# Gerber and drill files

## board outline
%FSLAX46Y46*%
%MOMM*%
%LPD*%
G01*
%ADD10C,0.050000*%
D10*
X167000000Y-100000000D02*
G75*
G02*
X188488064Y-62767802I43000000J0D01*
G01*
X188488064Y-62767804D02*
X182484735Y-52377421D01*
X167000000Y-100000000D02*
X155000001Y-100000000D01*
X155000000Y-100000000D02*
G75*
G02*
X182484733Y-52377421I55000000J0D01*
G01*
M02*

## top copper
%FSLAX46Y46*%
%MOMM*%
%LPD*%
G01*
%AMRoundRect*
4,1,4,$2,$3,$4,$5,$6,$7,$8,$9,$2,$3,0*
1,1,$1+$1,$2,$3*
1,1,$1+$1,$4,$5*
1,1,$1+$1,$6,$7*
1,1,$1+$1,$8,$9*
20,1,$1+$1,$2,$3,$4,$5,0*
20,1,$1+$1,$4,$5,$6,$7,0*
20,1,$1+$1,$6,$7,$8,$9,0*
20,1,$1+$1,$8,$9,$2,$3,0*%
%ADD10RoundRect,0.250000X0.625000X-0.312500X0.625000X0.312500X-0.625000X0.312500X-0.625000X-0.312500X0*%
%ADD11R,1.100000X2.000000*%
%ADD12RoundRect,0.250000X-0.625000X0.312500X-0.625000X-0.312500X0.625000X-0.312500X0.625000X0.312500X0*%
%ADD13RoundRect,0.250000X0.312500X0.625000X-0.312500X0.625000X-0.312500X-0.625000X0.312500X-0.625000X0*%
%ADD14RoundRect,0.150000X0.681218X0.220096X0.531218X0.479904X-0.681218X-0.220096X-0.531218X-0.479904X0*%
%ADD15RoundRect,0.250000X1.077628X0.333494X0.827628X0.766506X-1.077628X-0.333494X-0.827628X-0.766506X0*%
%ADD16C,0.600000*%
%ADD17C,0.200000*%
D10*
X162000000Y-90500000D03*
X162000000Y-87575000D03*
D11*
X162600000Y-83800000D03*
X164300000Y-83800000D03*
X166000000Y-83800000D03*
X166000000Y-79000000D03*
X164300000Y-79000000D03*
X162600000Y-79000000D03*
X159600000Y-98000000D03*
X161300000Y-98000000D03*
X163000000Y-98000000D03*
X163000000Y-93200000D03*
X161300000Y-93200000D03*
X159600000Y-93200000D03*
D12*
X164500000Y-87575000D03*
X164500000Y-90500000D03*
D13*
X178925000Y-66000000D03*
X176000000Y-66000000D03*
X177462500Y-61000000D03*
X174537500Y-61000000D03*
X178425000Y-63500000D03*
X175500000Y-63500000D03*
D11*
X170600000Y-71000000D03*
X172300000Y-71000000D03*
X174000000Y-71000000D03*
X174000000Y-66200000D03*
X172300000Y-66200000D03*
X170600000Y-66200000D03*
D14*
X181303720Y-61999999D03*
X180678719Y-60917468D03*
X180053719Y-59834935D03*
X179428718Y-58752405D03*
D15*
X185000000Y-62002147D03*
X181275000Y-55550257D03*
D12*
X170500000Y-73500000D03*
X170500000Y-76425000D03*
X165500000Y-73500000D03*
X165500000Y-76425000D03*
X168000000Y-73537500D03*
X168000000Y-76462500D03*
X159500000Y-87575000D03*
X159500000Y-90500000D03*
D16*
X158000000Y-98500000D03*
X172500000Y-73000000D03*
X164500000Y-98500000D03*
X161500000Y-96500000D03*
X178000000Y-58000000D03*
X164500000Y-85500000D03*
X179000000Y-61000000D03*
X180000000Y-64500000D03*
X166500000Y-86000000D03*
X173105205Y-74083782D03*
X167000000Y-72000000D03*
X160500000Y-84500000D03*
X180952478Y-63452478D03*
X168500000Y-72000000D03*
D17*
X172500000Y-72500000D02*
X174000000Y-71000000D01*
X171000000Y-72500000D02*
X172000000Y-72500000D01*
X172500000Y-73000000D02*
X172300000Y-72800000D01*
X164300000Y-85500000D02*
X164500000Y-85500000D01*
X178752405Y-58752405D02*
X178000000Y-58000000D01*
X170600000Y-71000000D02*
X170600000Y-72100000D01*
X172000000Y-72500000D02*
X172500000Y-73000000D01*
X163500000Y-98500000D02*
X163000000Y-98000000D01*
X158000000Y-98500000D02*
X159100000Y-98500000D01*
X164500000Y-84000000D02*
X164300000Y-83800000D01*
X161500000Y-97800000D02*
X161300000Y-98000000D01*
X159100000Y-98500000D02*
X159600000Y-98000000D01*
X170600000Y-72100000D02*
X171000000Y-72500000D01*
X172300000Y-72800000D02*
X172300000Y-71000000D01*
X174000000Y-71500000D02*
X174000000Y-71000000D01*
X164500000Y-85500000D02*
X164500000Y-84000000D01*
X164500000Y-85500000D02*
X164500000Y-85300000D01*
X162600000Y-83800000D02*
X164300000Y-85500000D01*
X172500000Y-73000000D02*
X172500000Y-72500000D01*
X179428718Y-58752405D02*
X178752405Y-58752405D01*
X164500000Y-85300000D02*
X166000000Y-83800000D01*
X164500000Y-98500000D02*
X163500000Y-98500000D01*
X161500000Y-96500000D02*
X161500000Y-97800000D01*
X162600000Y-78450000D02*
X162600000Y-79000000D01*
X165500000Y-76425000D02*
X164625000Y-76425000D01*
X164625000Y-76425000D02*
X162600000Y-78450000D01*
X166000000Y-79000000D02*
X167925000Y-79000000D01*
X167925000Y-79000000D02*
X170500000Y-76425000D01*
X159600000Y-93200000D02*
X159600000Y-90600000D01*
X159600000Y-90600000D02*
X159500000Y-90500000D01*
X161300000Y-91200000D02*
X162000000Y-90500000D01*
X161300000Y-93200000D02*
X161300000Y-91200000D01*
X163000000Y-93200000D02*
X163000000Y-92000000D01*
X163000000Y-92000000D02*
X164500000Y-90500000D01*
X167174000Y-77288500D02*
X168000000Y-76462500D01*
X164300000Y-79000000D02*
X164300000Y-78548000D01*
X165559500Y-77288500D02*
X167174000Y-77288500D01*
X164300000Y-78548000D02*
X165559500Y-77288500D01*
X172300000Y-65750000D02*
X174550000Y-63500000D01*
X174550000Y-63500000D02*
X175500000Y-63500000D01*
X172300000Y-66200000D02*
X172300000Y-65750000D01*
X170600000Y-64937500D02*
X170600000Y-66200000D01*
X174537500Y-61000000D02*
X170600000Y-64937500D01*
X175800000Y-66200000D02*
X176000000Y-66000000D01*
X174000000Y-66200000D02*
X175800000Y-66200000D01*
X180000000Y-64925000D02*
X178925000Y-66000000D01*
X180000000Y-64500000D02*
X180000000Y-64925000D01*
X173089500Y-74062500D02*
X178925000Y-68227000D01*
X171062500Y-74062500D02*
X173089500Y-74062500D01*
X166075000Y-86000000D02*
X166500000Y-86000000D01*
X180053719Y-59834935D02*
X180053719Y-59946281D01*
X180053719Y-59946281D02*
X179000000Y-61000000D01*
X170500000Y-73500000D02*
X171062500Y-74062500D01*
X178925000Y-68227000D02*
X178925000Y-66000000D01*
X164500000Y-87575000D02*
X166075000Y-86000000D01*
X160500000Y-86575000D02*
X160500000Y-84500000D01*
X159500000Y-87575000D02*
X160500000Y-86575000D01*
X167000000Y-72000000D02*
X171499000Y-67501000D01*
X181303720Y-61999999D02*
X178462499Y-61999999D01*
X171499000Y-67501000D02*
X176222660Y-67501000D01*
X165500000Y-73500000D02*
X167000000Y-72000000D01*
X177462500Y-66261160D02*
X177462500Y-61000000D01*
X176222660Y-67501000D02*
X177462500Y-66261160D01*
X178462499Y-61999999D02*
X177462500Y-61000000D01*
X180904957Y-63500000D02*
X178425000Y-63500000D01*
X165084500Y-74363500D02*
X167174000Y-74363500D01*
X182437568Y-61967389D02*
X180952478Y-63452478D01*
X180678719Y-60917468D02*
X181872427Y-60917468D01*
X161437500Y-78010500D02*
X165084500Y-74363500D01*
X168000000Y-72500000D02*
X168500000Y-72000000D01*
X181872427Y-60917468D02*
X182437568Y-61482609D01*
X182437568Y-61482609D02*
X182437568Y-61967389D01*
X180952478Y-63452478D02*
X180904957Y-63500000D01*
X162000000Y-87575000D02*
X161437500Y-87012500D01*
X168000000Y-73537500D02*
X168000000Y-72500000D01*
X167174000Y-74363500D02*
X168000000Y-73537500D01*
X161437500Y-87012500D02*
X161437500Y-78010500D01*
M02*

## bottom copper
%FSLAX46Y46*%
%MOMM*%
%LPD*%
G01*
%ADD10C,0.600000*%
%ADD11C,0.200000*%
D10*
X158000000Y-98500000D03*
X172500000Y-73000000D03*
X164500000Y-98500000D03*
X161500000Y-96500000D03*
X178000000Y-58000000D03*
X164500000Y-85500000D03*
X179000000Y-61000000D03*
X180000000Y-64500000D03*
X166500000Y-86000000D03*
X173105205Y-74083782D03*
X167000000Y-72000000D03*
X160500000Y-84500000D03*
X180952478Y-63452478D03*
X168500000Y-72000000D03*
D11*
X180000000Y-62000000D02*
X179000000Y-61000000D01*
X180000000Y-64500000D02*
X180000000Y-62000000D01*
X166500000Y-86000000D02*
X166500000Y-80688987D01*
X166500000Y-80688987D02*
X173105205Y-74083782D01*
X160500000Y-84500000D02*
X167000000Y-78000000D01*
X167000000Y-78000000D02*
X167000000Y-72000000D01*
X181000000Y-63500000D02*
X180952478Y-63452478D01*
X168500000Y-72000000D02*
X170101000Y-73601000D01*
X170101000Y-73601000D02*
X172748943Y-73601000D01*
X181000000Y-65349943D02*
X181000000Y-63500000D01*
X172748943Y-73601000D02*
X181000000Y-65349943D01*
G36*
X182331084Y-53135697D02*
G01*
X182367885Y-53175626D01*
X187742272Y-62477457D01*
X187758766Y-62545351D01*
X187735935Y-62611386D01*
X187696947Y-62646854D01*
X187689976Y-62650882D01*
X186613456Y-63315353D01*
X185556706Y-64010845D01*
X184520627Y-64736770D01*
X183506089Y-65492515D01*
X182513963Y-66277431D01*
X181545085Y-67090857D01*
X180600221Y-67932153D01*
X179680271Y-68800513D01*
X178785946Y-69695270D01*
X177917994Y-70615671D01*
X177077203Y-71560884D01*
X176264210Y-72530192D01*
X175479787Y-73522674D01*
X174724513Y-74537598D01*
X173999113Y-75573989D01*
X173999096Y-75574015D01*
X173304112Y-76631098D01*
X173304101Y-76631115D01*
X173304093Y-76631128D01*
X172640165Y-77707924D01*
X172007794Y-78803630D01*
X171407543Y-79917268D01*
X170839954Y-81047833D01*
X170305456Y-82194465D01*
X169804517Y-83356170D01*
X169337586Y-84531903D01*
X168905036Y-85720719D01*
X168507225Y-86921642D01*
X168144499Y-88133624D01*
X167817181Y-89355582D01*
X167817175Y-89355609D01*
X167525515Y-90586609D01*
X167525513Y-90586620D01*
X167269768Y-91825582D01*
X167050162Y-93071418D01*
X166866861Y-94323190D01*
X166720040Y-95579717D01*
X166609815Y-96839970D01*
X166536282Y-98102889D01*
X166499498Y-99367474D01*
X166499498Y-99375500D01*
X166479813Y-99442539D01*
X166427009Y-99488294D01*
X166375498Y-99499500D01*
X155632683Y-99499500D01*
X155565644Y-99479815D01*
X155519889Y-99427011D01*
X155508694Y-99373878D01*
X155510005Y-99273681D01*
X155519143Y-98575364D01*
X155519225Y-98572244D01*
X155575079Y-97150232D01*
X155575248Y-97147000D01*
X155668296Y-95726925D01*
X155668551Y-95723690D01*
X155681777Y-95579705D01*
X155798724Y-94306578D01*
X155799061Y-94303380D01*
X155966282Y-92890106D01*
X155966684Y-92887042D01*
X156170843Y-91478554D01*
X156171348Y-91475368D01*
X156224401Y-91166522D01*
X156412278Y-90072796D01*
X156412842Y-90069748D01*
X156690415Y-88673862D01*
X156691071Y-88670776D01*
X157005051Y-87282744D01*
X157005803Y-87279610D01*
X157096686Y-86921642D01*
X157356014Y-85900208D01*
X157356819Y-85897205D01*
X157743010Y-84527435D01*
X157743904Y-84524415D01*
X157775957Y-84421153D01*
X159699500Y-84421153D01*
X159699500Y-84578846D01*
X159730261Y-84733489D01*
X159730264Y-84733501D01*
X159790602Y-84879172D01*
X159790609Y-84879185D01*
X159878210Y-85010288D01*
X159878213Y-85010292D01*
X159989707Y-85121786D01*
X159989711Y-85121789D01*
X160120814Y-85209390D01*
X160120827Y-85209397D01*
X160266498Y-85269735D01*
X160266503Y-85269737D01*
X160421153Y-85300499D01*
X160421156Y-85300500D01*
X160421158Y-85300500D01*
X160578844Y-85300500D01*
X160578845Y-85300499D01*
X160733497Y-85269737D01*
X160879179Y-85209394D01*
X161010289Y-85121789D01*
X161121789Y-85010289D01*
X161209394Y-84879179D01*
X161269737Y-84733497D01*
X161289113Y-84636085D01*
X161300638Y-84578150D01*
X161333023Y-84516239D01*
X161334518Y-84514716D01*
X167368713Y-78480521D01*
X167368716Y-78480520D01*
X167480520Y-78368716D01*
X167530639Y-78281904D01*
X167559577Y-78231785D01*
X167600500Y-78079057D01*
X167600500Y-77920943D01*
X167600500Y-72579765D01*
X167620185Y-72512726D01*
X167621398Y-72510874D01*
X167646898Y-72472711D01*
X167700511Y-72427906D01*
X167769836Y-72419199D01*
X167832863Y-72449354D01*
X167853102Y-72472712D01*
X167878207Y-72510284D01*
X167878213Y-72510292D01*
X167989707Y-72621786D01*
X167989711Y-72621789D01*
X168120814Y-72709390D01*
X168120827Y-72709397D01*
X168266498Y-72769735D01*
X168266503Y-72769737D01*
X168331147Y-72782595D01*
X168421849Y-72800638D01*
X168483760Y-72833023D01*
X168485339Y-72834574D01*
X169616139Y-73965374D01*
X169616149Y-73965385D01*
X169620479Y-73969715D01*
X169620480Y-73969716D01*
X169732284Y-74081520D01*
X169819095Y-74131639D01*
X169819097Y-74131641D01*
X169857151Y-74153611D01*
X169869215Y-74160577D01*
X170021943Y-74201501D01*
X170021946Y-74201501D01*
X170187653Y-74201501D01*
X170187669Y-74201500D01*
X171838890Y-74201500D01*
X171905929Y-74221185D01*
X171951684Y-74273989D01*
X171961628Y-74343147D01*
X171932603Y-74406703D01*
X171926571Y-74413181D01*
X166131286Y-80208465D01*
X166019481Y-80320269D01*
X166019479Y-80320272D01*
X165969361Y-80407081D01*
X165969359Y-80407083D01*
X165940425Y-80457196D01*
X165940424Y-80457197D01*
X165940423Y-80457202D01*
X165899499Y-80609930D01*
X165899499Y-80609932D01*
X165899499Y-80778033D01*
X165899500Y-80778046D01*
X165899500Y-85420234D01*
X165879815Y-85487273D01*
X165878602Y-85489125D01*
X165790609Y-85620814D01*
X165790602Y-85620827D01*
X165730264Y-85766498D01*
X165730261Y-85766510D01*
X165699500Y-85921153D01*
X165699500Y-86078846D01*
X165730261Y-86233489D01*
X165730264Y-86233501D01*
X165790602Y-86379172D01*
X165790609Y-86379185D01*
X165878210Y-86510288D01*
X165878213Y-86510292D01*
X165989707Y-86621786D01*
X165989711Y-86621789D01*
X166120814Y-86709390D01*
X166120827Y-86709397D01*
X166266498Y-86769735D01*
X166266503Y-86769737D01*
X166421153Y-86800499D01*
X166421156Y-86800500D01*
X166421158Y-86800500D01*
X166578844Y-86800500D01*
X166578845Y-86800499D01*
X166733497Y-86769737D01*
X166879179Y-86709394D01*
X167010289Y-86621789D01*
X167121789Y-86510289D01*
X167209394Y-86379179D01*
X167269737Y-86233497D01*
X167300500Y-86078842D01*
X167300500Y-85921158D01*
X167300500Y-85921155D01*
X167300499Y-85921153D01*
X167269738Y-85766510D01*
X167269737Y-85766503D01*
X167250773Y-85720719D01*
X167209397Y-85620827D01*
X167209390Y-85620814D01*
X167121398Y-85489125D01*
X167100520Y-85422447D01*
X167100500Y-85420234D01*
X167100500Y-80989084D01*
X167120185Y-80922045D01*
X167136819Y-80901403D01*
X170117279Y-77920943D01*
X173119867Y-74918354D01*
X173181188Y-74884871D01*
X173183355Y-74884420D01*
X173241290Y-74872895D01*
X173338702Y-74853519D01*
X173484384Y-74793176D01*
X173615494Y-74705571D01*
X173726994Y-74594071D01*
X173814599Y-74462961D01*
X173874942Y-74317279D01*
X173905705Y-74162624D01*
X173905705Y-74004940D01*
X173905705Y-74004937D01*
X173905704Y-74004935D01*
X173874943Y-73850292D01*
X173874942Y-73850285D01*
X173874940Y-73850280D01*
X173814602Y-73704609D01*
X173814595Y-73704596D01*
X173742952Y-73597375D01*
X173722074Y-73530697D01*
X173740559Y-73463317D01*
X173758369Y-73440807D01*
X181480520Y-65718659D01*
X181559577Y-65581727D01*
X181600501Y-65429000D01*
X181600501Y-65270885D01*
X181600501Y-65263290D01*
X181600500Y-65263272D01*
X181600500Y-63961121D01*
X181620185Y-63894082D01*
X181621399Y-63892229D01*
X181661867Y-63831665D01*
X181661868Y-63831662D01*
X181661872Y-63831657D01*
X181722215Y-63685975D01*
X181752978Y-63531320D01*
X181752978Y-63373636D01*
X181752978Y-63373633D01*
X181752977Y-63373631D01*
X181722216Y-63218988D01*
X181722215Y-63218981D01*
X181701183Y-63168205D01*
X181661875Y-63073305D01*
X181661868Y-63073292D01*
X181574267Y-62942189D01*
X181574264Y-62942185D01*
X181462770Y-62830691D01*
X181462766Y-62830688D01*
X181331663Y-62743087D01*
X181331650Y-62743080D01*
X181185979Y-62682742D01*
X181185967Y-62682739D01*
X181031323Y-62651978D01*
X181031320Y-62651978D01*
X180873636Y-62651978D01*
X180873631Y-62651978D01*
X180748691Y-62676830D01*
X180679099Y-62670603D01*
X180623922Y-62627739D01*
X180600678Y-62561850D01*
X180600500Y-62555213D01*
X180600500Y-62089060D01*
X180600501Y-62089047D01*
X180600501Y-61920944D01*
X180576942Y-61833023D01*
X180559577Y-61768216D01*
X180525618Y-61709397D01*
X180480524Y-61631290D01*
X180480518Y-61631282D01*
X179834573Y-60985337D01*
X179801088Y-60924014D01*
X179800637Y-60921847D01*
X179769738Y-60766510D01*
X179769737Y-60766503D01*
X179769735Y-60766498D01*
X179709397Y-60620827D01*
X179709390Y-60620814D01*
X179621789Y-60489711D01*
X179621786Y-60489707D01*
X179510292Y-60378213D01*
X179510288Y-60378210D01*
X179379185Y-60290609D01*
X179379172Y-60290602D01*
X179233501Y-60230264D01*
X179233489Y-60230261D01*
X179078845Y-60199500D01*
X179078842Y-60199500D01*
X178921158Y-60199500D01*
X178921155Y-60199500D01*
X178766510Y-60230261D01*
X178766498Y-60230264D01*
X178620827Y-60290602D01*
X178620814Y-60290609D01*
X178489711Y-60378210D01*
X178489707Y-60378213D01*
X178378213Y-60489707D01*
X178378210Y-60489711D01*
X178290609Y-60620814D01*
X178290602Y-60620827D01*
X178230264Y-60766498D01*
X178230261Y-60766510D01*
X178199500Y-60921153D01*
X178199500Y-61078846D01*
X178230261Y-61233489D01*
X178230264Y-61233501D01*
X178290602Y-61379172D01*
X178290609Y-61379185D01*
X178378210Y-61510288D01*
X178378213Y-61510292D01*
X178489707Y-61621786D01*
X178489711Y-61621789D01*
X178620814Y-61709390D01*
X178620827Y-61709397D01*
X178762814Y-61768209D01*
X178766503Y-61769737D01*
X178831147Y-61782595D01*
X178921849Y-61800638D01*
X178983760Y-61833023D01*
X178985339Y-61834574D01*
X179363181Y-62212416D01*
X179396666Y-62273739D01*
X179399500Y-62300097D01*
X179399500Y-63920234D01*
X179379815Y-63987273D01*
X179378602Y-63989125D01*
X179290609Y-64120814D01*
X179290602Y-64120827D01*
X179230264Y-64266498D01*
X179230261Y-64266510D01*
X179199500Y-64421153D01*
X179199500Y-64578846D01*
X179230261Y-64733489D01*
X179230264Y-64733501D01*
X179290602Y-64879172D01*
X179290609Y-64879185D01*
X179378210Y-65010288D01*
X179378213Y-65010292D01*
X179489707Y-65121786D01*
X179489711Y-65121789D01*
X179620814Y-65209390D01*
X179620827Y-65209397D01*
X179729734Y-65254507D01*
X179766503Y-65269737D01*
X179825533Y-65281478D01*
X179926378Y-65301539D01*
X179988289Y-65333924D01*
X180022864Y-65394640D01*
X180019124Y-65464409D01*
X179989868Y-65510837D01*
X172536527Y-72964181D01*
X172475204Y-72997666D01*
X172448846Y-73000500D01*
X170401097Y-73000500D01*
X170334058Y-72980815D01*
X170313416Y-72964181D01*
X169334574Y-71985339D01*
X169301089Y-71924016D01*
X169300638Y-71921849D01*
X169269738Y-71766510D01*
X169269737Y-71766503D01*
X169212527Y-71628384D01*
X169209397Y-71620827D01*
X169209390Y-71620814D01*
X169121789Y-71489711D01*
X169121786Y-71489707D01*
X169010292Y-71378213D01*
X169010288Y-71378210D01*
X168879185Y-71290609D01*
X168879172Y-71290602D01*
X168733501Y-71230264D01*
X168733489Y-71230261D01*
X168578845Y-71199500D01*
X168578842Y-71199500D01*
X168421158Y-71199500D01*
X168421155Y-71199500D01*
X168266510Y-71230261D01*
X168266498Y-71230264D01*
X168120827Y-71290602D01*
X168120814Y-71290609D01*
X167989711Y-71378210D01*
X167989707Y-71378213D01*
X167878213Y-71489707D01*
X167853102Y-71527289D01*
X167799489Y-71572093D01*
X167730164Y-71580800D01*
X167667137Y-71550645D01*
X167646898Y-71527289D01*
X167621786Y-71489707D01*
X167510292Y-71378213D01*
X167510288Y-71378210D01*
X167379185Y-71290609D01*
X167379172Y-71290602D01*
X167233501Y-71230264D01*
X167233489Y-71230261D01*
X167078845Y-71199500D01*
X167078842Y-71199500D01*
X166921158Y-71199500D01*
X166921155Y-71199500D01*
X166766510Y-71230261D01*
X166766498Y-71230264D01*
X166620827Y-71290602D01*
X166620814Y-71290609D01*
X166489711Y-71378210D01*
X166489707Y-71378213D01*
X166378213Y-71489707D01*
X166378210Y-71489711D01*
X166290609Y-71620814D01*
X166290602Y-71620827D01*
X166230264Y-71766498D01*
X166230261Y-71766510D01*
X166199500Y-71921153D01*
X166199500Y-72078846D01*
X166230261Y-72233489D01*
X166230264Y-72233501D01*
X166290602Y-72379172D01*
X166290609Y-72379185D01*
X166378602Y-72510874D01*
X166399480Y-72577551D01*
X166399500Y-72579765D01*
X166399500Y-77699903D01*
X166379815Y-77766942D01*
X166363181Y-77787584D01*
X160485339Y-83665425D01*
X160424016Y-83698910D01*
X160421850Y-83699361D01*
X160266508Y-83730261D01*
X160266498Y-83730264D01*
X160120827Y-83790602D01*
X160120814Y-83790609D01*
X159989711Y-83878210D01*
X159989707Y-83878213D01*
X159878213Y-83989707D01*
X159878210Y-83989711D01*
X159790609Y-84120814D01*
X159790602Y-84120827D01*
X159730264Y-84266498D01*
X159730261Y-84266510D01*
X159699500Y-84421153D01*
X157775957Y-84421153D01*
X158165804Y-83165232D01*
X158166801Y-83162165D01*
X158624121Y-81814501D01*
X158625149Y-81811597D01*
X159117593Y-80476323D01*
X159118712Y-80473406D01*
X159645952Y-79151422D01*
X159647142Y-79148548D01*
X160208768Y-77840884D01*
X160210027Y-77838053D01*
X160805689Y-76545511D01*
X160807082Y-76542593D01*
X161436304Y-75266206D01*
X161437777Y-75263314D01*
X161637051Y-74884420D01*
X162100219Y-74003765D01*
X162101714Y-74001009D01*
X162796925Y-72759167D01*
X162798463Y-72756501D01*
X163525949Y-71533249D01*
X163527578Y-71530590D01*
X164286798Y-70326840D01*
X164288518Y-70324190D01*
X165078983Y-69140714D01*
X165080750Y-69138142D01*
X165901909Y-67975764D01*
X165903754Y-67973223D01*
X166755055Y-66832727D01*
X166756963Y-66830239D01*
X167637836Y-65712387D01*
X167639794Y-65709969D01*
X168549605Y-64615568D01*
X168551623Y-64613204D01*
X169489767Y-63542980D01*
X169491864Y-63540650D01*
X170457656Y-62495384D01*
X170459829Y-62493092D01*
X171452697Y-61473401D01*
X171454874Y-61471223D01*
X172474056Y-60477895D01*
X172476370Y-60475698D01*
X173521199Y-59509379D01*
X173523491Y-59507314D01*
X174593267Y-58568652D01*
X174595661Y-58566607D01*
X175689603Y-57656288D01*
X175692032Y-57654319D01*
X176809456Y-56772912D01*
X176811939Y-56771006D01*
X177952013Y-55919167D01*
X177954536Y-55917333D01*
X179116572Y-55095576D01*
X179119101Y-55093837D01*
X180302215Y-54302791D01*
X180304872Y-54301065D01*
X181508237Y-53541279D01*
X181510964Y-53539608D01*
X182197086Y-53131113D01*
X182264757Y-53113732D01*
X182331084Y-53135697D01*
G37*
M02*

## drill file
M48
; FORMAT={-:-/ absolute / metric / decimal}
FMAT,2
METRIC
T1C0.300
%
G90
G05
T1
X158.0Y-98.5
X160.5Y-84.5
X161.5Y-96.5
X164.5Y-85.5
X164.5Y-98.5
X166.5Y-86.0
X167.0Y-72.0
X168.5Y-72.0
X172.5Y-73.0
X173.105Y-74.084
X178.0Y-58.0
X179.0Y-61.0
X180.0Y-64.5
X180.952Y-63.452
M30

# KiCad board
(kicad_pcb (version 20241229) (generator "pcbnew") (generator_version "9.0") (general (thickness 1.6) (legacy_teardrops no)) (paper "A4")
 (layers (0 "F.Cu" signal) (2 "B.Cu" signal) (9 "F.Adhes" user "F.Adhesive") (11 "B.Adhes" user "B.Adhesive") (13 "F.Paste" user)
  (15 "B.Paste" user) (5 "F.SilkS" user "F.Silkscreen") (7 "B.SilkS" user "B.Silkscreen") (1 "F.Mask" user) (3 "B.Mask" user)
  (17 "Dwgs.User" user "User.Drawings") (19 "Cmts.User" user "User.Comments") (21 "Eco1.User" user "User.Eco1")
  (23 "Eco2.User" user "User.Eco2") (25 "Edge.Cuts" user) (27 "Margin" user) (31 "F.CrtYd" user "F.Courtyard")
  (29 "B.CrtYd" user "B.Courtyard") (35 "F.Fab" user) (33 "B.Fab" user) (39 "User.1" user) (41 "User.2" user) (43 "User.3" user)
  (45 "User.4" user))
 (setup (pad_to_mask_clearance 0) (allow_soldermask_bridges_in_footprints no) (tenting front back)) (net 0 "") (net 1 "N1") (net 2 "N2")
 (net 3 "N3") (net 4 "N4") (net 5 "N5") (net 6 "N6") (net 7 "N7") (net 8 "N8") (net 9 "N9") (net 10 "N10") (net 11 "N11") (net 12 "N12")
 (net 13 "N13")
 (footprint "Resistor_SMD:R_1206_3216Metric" (layer "F.Cu") (at 162 89.0375 90)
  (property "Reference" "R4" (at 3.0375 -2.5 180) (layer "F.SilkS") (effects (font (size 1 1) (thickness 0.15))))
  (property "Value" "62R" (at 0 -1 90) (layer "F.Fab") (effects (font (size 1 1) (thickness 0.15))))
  (pad "1" smd roundrect (at -1.4625 0 90) (size 1.125 1.75) (layers "F.Cu" "F.Mask" "F.Paste") (roundrect_rratio 0.222222) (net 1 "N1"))
  (pad "2" smd roundrect (at 1.4625 0 90) (size 1.125 1.75) (layers "F.Cu" "F.Mask" "F.Paste") (roundrect_rratio 0.222222) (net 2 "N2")))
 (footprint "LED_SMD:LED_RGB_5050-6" (layer "F.Cu") (at 164.3 81.4 90)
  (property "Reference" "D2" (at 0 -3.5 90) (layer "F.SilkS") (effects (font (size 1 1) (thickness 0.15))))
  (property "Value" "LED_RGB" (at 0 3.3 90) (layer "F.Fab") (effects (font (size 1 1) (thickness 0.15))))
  (pad "1" smd rect (at -2.4 -1.7 180) (size 1.1 2) (layers "F.Cu" "F.Mask" "F.Paste") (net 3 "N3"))
  (pad "2" smd rect (at -2.4 0 180) (size 1.1 2) (layers "F.Cu" "F.Mask" "F.Paste") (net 3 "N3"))
  (pad "3" smd rect (at -2.4 1.7 180) (size 1.1 2) (layers "F.Cu" "F.Mask" "F.Paste") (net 3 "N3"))
  (pad "4" smd rect (at 2.4 1.7 180) (size 1.1 2) (layers "F.Cu" "F.Mask" "F.Paste") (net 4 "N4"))
  (pad "5" smd rect (at 2.4 0 180) (size 1.1 2) (layers "F.Cu" "F.Mask" "F.Paste") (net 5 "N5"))
  (pad "6" smd rect (at 2.4 -1.7 180) (size 1.1 2) (layers "F.Cu" "F.Mask" "F.Paste") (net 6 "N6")))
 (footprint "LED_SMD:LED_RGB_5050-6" (layer "F.Cu") (at 161.3 95.6 90)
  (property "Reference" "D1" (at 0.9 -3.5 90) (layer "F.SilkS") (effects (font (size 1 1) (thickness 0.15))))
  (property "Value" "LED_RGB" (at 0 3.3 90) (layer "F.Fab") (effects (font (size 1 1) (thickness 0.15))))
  (pad "1" smd rect (at -2.4 -1.7 180) (size 1.1 2) (layers "F.Cu" "F.Mask" "F.Paste") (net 3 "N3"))
  (pad "2" smd rect (at -2.4 0 180) (size 1.1 2) (layers "F.Cu" "F.Mask" "F.Paste") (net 3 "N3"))
  (pad "3" smd rect (at -2.4 1.7 180) (size 1.1 2) (layers "F.Cu" "F.Mask" "F.Paste") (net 3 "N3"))
  (pad "4" smd rect (at 2.4 1.7 180) (size 1.1 2) (layers "F.Cu" "F.Mask" "F.Paste") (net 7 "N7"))
  (pad "5" smd rect (at 2.4 0 180) (size 1.1 2) (layers "F.Cu" "F.Mask" "F.Paste") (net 1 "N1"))
  (pad "6" smd rect (at 2.4 -1.7 180) (size 1.1 2) (layers "F.Cu" "F.Mask" "F.Paste") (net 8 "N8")))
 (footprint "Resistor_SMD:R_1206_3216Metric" (layer "F.Cu") (at 164.5 89.0375 -90)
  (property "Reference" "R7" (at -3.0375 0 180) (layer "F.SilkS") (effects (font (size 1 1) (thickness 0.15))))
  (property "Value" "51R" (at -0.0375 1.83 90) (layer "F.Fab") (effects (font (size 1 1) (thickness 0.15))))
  (pad "1" smd roundrect (at -1.4625 0 270) (size 1.125 1.75) (layers "F.Cu" "F.Mask" "F.Paste") (roundrect_rratio 0.222222) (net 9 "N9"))
  (pad "2" smd roundrect (at 1.4625 0 270) (size 1.125 1.75) (layers "F.Cu" "F.Mask" "F.Paste") (roundrect_rratio 0.222222) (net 7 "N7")))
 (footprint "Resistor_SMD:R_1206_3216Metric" (layer "F.Cu") (at 177.4625 66 180)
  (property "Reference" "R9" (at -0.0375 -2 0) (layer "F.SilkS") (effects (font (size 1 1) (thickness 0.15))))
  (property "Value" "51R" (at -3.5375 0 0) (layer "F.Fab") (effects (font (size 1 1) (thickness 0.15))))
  (pad "1" smd roundrect (at -1.4625 0 180) (size 1.125 1.75) (layers "F.Cu" "F.Mask" "F.Paste") (roundrect_rratio 0.222222) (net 9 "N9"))
  (pad "2" smd roundrect (at 1.4625 0 180) (size 1.125 1.75) (layers "F.Cu" "F.Mask" "F.Paste") (roundrect_rratio 0.222222) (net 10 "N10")))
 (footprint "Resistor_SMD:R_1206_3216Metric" (layer "F.Cu") (at 176 61 180)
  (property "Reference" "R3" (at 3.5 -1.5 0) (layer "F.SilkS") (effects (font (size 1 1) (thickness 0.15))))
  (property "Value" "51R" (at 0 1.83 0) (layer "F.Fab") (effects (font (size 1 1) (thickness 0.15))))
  (pad "1" smd roundrect (at -1.4625 0 180) (size 1.125 1.75) (layers "F.Cu" "F.Mask" "F.Paste") (roundrect_rratio 0.222222) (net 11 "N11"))
  (pad "2" smd roundrect (at 1.4625 0 180) (size 1.125 1.75) (layers "F.Cu" "F.Mask" "F.Paste") (roundrect_rratio 0.222222) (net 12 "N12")))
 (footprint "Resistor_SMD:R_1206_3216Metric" (layer "F.Cu") (at 176.9625 63.5 180)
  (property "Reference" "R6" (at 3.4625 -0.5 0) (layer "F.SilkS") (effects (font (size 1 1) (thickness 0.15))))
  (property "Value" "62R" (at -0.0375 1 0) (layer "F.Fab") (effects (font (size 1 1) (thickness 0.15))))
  (pad "1" smd roundrect (at -1.4625 0 180) (size 1.125 1.75) (layers "F.Cu" "F.Mask" "F.Paste") (roundrect_rratio 0.222222) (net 2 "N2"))
  (pad "2" smd roundrect (at 1.4625 0 180) (size 1.125 1.75) (layers "F.Cu" "F.Mask" "F.Paste") (roundrect_rratio 0.222222) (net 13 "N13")))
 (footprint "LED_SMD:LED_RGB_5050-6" (layer "F.Cu") (at 172.3 68.6 90)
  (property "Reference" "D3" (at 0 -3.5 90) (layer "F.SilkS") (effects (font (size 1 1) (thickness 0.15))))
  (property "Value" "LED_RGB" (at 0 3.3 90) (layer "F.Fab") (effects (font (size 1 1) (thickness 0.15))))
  (pad "1" smd rect (at -2.4 -1.7 180) (size 1.1 2) (layers "F.Cu" "F.Mask" "F.Paste") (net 3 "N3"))
  (pad "2" smd rect (at -2.4 0 180) (size 1.1 2) (layers "F.Cu" "F.Mask" "F.Paste") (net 3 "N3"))
  (pad "3" smd rect (at -2.4 1.7 180) (size 1.1 2) (layers "F.Cu" "F.Mask" "F.Paste") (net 3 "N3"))
  (pad "4" smd rect (at 2.4 1.7 180) (size 1.1 2) (layers "F.Cu" "F.Mask" "F.Paste") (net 10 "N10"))
  (pad "5" smd rect (at 2.4 0 180) (size 1.1 2) (layers "F.Cu" "F.Mask" "F.Paste") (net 13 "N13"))
  (pad "6" smd rect (at 2.4 -1.7 180) (size 1.1 2) (layers "F.Cu" "F.Mask" "F.Paste") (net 12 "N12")))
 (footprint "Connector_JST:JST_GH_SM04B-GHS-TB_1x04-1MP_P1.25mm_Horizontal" (layer "F.Cu") (at 181.968366 59.451202 120)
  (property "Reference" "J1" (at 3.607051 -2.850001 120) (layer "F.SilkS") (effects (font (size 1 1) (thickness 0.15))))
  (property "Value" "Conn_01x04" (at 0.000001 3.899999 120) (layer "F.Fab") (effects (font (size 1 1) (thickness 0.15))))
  (pad "1" smd roundrect (at -1.875 -1.849999 120) (size 0.6 1.7) (layers "F.Cu" "F.Mask" "F.Paste") (roundrect_rratio 0.25) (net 11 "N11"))
  (pad "2" smd roundrect (at -0.625 -1.85 120) (size 0.6 1.7) (layers "F.Cu" "F.Mask" "F.Paste") (roundrect_rratio 0.25) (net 2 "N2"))
  (pad "3" smd roundrect (at 0.625001 -1.849999 120) (size 0.6 1.7) (layers "F.Cu" "F.Mask" "F.Paste") (roundrect_rratio 0.25) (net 9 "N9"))
  (pad "4" smd roundrect (at 1.875 -1.850001 120) (size 0.6 1.7) (layers "F.Cu" "F.Mask" "F.Paste") (roundrect_rratio 0.25) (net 3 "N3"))
  (pad "MP" smd roundrect (at -3.725 1.35 120) (size 1 2.7) (layers "F.Cu" "F.Mask" "F.Paste") (roundrect_rratio 0.25))
  (pad "MP" smd roundrect (at 3.725 1.35 120) (size 1 2.7) (layers "F.Cu" "F.Mask" "F.Paste") (roundrect_rratio 0.25)))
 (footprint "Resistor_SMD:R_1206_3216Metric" (layer "F.Cu") (at 170.5 74.9625 -90)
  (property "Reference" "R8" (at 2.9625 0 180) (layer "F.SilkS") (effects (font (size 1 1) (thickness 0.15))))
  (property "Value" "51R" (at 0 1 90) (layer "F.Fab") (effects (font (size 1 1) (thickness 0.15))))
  (pad "1" smd roundrect (at -1.4625 0 270) (size 1.125 1.75) (layers "F.Cu" "F.Mask" "F.Paste") (roundrect_rratio 0.222222) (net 9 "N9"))
  (pad "2" smd roundrect (at 1.4625 0 270) (size 1.125 1.75) (layers "F.Cu" "F.Mask" "F.Paste") (roundrect_rratio 0.222222) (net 4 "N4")))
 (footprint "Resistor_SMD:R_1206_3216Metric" (layer "F.Cu") (at 165.5 74.9625 -90)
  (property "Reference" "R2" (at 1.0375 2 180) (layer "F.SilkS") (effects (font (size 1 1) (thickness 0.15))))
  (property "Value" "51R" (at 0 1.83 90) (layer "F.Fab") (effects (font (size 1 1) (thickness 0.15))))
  (pad "1" smd roundrect (at -1.4625 0 270) (size 1.125 1.75) (layers "F.Cu" "F.Mask" "F.Paste") (roundrect_rratio 0.222222) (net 11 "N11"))
  (pad "2" smd roundrect (at 1.4625 0 270) (size 1.125 1.75) (layers "F.Cu" "F.Mask" "F.Paste") (roundrect_rratio 0.222222) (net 6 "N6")))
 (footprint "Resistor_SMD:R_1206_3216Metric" (layer "F.Cu") (at 168 75 -90)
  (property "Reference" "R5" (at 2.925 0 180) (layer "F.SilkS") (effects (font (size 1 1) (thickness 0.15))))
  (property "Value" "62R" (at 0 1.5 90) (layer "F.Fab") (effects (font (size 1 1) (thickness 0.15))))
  (pad "1" smd roundrect (at -1.4625 0 270) (size 1.125 1.75) (layers "F.Cu" "F.Mask" "F.Paste") (roundrect_rratio 0.222222) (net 2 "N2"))
  (pad "2" smd roundrect (at 1.4625 0 270) (size 1.125 1.75) (layers "F.Cu" "F.Mask" "F.Paste") (roundrect_rratio 0.222222) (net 5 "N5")))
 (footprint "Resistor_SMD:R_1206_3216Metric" (layer "F.Cu") (at 159.5 89.0375 -90)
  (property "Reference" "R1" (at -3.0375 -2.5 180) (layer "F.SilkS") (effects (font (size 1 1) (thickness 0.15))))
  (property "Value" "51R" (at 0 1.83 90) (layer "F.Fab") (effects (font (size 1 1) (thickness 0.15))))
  (pad "1" smd roundrect (at -1.4625 0 270) (size 1.125 1.75) (layers "F.Cu" "F.Mask" "F.Paste") (roundrect_rratio 0.222222) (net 11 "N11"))
  (pad "2" smd roundrect (at 1.4625 0 270) (size 1.125 1.75) (layers "F.Cu" "F.Mask" "F.Paste") (roundrect_rratio 0.222222) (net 8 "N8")))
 (gr_arc (start 167 100) (mid 172.757462 78.505969) (end 188.488064 62.767802) (stroke (width 0.05) (type default)) (layer "Edge.Cuts"))
 (gr_line (start 188.488064 62.767804) (end 182.484735 52.377421) (stroke (width 0.05) (type default)) (layer "Edge.Cuts"))
 (gr_line (start 167 100) (end 155.000001 100) (stroke (width 0.05) (type default)) (layer "Edge.Cuts"))
 (gr_arc (start 155 100) (mid 162.364196 72.507635) (end 182.484733 52.377421) (stroke (width 0.05) (type default)) (layer "Edge.Cuts"))
 (segment (start 172.5 72.5) (end 174 71) (width 0.2) (layer "F.Cu") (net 3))
 (segment (start 171 72.5) (end 172 72.5) (width 0.2) (layer "F.Cu") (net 3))
 (segment (start 172.5 73) (end 172.3 72.8) (width 0.2) (layer "F.Cu") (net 3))
 (segment (start 164.3 85.5) (end 164.5 85.5) (width 0.2) (layer "F.Cu") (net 3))
 (segment (start 178.752405 58.752405) (end 178 58) (width 0.2) (layer "F.Cu") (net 3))
 (segment (start 170.6 71) (end 170.6 72.1) (width 0.2) (layer "F.Cu") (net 3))
 (segment (start 172 72.5) (end 172.5 73) (width 0.2) (layer "F.Cu") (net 3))
 (segment (start 163.5 98.5) (end 163 98) (width 0.2) (layer "F.Cu") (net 3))
 (segment (start 158 98.5) (end 159.1 98.5) (width 0.2) (layer "F.Cu") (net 3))
 (segment (start 164.5 84) (end 164.3 83.8) (width 0.2) (layer "F.Cu") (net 3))
 (segment (start 161.5 97.8) (end 161.3 98) (width 0.2) (layer "F.Cu") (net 3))
 (segment (start 159.1 98.5) (end 159.6 98) (width 0.2) (layer "F.Cu") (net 3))
 (segment (start 170.6 72.1) (end 171 72.5) (width 0.2) (layer "F.Cu") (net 3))
 (segment (start 172.3 72.8) (end 172.3 71) (width 0.2) (layer "F.Cu") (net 3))
 (segment (start 174 71.5) (end 174 71) (width 0.2) (layer "F.Cu") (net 3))
 (segment (start 164.5 85.5) (end 164.5 84) (width 0.2) (layer "F.Cu") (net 3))
 (segment (start 164.5 85.5) (end 164.5 85.3) (width 0.2) (layer "F.Cu") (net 3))
 (segment (start 162.6 83.8) (end 164.3 85.5) (width 0.2) (layer "F.Cu") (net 3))
 (segment (start 172.5 73) (end 172.5 72.5) (width 0.2) (layer "F.Cu") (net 3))
 (segment (start 179.428718 58.752405) (end 178.752405 58.752405) (width 0.2) (layer "F.Cu") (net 3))
 (segment (start 164.5 85.3) (end 166 83.8) (width 0.2) (layer "F.Cu") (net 3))
 (segment (start 164.5 98.5) (end 163.5 98.5) (width 0.2) (layer "F.Cu") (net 3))
 (segment (start 161.5 96.5) (end 161.5 97.8) (width 0.2) (layer "F.Cu") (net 3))
 (via (at 158 98.5) (size 0.6) (drill 0.3) (layers "F.Cu" "B.Cu") (free yes) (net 3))
 (via (at 172.5 73) (size 0.6) (drill 0.3) (layers "F.Cu" "B.Cu") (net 3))
 (via (at 164.5 98.5) (size 0.6) (drill 0.3) (layers "F.Cu" "B.Cu") (free yes) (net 3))
 (via (at 161.5 96.5) (size 0.6) (drill 0.3) (layers "F.Cu" "B.Cu") (free yes) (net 3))
 (via (at 178 58) (size 0.6) (drill 0.3) (layers "F.Cu" "B.Cu") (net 3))
 (via (at 164.5 85.5) (size 0.6) (drill 0.3) (layers "F.Cu" "B.Cu") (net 3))
 (segment (start 162.6 78.45) (end 162.6 79) (width 0.2) (layer "F.Cu") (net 6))
 (segment (start 165.5 76.425) (end 164.625 76.425) (width 0.2) (layer "F.Cu") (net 6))
 (segment (start 164.625 76.425) (end 162.6 78.45) (width 0.2) (layer "F.Cu") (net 6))
 (segment (start 166 79) (end 167.925 79) (width 0.2) (layer "F.Cu") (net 4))
 (segment (start 167.925 79) (end 170.5 76.425) (width 0.2) (layer "F.Cu") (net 4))
 (segment (start 159.6 93.2) (end 159.6 90.6) (width 0.2) (layer "F.Cu") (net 8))
 (segment (start 159.6 90.6) (end 159.5 90.5) (width 0.2) (layer "F.Cu") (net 8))
 (segment (start 161.3 91.2) (end 162 90.5) (width 0.2) (layer "F.Cu") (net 1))
 (segment (start 161.3 93.2) (end 161.3 91.2) (width 0.2) (layer "F.Cu") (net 1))
 (segment (start 163 93.2) (end 163 92) (width 0.2) (layer "F.Cu") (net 7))
 (segment (start 163 92) (end 164.5 90.5) (width 0.2) (layer "F.Cu") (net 7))
 (segment (start 167.174 77.2885) (end 168 76.4625) (width 0.2) (layer "F.Cu") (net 5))
 (segment (start 164.3 79) (end 164.3 78.548) (width 0.2) (layer "F.Cu") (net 5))
 (segment (start 165.5595 77.2885) (end 167.174 77.2885) (width 0.2) (layer "F.Cu") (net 5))
 (segment (start 164.3 78.548) (end 165.5595 77.2885) (width 0.2) (layer "F.Cu") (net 5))
 (segment (start 172.3 65.75) (end 174.55 63.5) (width 0.2) (layer "F.Cu") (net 13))
 (segment (start 174.55 63.5) (end 175.5 63.5) (width 0.2) (layer "F.Cu") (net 13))
 (segment (start 172.3 66.2) (end 172.3 65.75) (width 0.2) (layer "F.Cu") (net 13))
 (segment (start 170.6 64.9375) (end 170.6 66.2) (width 0.2) (layer "F.Cu") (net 12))
 (segment (start 174.5375 61) (end 170.6 64.9375) (width 0.2) (layer "F.Cu") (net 12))
 (segment (start 175.8 66.2) (end 176 66) (width 0.2) (layer "F.Cu") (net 10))
 (segment (start 174 66.2) (end 175.8 66.2) (width 0.2) (layer "F.Cu") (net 10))
 (segment (start 180 64.925) (end 178.925 66) (width 0.2) (layer "F.Cu") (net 9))
 (segment (start 180 64.5) (end 180 64.925) (width 0.2) (layer "F.Cu") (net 9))
 (segment (start 173.0895 74.0625) (end 178.925 68.227) (width 0.2) (layer "F.Cu") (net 9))
 (segment (start 171.0625 74.0625) (end 173.0895 74.0625) (width 0.2) (layer "F.Cu") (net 9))
 (segment (start 166.075 86) (end 166.5 86) (width 0.2) (layer "F.Cu") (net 9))
 (segment (start 180.053719 59.834935) (end 180.053719 59.946281) (width 0.2) (layer "F.Cu") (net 9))
 (segment (start 180.053719 59.946281) (end 179 61) (width 0.2) (layer "F.Cu") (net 9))
 (segment (start 170.5 73.5) (end 171.0625 74.0625) (width 0.2) (layer "F.Cu") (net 9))
 (segment (start 178.925 68.227) (end 178.925 66) (width 0.2) (layer "F.Cu") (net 9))
 (segment (start 164.5 87.575) (end 166.075 86) (width 0.2) (layer "F.Cu") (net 9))
 (via (at 179 61) (size 0.6) (drill 0.3) (layers "F.Cu" "B.Cu") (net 9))
 (via (at 180 64.5) (size 0.6) (drill 0.3) (layers "F.Cu" "B.Cu") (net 9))
 (via (at 166.5 86) (size 0.6) (drill 0.3) (layers "F.Cu" "B.Cu") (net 9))
 (via (at 173.105205 74.083782) (size 0.6) (drill 0.3) (layers "F.Cu" "B.Cu") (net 9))
 (segment (start 180 62) (end 179 61) (width 0.2) (layer "B.Cu") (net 9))
 (segment (start 180 64.5) (end 180 62) (width 0.2) (layer "B.Cu") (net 9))
 (segment (start 166.5 86) (end 166.5 80.688987) (width 0.2) (layer "B.Cu") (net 9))
 (segment (start 166.5 80.688987) (end 173.105205 74.083782) (width 0.2) (layer "B.Cu") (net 9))
 (segment (start 160.5 86.575) (end 160.5 84.5) (width 0.2) (layer "F.Cu") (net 11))
 (segment (start 159.5 87.575) (end 160.5 86.575) (width 0.2) (layer "F.Cu") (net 11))
 (segment (start 167 72) (end 171.499 67.501) (width 0.2) (layer "F.Cu") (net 11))
 (segment (start 181.30372 61.999999) (end 178.462499 61.999999) (width 0.2) (layer "F.Cu") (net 11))
 (segment (start 171.499 67.501) (end 176.22266 67.501) (width 0.2) (layer "F.Cu") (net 11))
 (segment (start 165.5 73.5) (end 167 72) (width 0.2) (layer "F.Cu") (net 11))
 (segment (start 177.4625 66.26116) (end 177.4625 61) (width 0.2) (layer "F.Cu") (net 11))
 (segment (start 176.22266 67.501) (end 177.4625 66.26116) (width 0.2) (layer "F.Cu") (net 11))
 (segment (start 178.462499 61.999999) (end 177.4625 61) (width 0.2) (layer "F.Cu") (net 11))
 (via (at 167 72) (size 0.6) (drill 0.3) (layers "F.Cu" "B.Cu") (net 11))
 (via (at 160.5 84.5) (size 0.6) (drill 0.3) (layers "F.Cu" "B.Cu") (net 11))
 (segment (start 160.5 84.5) (end 167 78) (width 0.2) (layer "B.Cu") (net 11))
 (segment (start 167 78) (end 167 72) (width 0.2) (layer "B.Cu") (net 11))
 (segment (start 180.904957 63.5) (end 178.425 63.5) (width 0.2) (layer "F.Cu") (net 2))
 (segment (start 165.0845 74.3635) (end 167.174 74.3635) (width 0.2) (layer "F.Cu") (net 2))
 (segment (start 182.437568 61.967389) (end 180.952478 63.452478) (width 0.2) (layer "F.Cu") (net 2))
 (segment (start 180.678719 60.917468) (end 181.872427 60.917468) (width 0.2) (layer "F.Cu") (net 2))
 (segment (start 161.4375 78.0105) (end 165.0845 74.3635) (width 0.2) (layer "F.Cu") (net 2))
 (segment (start 168 72.5) (end 168.5 72) (width 0.2) (layer "F.Cu") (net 2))
 (segment (start 181.872427 60.917468) (end 182.437568 61.482609) (width 0.2) (layer "F.Cu") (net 2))
 (segment (start 182.437568 61.482609) (end 182.437568 61.967389) (width 0.2) (layer "F.Cu") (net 2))
 (segment (start 180.952478 63.452478) (end 180.904957 63.5) (width 0.2) (layer "F.Cu") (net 2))
 (segment (start 162 87.575) (end 161.4375 87.0125) (width 0.2) (layer "F.Cu") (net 2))
 (segment (start 168 73.5375) (end 168 72.5) (width 0.2) (layer "F.Cu") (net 2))
 (segment (start 167.174 74.3635) (end 168 73.5375) (width 0.2) (layer "F.Cu") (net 2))
 (segment (start 161.4375 87.0125) (end 161.4375 78.0105) (width 0.2) (layer "F.Cu") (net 2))
 (via (at 180.952478 63.452478) (size 0.6) (drill 0.3) (layers "F.Cu" "B.Cu") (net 2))
 (via (at 168.5 72) (size 0.6) (drill 0.3) (layers "F.Cu" "B.Cu") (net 2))
 (segment (start 181 63.5) (end 180.952478 63.452478) (width 0.2) (layer "B.Cu") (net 2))
 (segment (start 168.5 72) (end 170.101 73.601) (width 0.2) (layer "B.Cu") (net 2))
 (segment (start 170.101 73.601) (end 172.748943 73.601) (width 0.2) (layer "B.Cu") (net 2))
 (segment (start 181 65.349943) (end 181 63.5) (width 0.2) (layer "B.Cu") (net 2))
 (segment (start 172.748943 73.601) (end 181 65.349943) (width 0.2) (layer "B.Cu") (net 2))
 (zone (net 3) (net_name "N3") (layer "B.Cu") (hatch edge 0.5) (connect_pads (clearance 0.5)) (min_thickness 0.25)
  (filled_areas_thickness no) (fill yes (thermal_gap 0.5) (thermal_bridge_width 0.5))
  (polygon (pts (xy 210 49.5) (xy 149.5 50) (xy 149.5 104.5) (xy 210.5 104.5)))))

